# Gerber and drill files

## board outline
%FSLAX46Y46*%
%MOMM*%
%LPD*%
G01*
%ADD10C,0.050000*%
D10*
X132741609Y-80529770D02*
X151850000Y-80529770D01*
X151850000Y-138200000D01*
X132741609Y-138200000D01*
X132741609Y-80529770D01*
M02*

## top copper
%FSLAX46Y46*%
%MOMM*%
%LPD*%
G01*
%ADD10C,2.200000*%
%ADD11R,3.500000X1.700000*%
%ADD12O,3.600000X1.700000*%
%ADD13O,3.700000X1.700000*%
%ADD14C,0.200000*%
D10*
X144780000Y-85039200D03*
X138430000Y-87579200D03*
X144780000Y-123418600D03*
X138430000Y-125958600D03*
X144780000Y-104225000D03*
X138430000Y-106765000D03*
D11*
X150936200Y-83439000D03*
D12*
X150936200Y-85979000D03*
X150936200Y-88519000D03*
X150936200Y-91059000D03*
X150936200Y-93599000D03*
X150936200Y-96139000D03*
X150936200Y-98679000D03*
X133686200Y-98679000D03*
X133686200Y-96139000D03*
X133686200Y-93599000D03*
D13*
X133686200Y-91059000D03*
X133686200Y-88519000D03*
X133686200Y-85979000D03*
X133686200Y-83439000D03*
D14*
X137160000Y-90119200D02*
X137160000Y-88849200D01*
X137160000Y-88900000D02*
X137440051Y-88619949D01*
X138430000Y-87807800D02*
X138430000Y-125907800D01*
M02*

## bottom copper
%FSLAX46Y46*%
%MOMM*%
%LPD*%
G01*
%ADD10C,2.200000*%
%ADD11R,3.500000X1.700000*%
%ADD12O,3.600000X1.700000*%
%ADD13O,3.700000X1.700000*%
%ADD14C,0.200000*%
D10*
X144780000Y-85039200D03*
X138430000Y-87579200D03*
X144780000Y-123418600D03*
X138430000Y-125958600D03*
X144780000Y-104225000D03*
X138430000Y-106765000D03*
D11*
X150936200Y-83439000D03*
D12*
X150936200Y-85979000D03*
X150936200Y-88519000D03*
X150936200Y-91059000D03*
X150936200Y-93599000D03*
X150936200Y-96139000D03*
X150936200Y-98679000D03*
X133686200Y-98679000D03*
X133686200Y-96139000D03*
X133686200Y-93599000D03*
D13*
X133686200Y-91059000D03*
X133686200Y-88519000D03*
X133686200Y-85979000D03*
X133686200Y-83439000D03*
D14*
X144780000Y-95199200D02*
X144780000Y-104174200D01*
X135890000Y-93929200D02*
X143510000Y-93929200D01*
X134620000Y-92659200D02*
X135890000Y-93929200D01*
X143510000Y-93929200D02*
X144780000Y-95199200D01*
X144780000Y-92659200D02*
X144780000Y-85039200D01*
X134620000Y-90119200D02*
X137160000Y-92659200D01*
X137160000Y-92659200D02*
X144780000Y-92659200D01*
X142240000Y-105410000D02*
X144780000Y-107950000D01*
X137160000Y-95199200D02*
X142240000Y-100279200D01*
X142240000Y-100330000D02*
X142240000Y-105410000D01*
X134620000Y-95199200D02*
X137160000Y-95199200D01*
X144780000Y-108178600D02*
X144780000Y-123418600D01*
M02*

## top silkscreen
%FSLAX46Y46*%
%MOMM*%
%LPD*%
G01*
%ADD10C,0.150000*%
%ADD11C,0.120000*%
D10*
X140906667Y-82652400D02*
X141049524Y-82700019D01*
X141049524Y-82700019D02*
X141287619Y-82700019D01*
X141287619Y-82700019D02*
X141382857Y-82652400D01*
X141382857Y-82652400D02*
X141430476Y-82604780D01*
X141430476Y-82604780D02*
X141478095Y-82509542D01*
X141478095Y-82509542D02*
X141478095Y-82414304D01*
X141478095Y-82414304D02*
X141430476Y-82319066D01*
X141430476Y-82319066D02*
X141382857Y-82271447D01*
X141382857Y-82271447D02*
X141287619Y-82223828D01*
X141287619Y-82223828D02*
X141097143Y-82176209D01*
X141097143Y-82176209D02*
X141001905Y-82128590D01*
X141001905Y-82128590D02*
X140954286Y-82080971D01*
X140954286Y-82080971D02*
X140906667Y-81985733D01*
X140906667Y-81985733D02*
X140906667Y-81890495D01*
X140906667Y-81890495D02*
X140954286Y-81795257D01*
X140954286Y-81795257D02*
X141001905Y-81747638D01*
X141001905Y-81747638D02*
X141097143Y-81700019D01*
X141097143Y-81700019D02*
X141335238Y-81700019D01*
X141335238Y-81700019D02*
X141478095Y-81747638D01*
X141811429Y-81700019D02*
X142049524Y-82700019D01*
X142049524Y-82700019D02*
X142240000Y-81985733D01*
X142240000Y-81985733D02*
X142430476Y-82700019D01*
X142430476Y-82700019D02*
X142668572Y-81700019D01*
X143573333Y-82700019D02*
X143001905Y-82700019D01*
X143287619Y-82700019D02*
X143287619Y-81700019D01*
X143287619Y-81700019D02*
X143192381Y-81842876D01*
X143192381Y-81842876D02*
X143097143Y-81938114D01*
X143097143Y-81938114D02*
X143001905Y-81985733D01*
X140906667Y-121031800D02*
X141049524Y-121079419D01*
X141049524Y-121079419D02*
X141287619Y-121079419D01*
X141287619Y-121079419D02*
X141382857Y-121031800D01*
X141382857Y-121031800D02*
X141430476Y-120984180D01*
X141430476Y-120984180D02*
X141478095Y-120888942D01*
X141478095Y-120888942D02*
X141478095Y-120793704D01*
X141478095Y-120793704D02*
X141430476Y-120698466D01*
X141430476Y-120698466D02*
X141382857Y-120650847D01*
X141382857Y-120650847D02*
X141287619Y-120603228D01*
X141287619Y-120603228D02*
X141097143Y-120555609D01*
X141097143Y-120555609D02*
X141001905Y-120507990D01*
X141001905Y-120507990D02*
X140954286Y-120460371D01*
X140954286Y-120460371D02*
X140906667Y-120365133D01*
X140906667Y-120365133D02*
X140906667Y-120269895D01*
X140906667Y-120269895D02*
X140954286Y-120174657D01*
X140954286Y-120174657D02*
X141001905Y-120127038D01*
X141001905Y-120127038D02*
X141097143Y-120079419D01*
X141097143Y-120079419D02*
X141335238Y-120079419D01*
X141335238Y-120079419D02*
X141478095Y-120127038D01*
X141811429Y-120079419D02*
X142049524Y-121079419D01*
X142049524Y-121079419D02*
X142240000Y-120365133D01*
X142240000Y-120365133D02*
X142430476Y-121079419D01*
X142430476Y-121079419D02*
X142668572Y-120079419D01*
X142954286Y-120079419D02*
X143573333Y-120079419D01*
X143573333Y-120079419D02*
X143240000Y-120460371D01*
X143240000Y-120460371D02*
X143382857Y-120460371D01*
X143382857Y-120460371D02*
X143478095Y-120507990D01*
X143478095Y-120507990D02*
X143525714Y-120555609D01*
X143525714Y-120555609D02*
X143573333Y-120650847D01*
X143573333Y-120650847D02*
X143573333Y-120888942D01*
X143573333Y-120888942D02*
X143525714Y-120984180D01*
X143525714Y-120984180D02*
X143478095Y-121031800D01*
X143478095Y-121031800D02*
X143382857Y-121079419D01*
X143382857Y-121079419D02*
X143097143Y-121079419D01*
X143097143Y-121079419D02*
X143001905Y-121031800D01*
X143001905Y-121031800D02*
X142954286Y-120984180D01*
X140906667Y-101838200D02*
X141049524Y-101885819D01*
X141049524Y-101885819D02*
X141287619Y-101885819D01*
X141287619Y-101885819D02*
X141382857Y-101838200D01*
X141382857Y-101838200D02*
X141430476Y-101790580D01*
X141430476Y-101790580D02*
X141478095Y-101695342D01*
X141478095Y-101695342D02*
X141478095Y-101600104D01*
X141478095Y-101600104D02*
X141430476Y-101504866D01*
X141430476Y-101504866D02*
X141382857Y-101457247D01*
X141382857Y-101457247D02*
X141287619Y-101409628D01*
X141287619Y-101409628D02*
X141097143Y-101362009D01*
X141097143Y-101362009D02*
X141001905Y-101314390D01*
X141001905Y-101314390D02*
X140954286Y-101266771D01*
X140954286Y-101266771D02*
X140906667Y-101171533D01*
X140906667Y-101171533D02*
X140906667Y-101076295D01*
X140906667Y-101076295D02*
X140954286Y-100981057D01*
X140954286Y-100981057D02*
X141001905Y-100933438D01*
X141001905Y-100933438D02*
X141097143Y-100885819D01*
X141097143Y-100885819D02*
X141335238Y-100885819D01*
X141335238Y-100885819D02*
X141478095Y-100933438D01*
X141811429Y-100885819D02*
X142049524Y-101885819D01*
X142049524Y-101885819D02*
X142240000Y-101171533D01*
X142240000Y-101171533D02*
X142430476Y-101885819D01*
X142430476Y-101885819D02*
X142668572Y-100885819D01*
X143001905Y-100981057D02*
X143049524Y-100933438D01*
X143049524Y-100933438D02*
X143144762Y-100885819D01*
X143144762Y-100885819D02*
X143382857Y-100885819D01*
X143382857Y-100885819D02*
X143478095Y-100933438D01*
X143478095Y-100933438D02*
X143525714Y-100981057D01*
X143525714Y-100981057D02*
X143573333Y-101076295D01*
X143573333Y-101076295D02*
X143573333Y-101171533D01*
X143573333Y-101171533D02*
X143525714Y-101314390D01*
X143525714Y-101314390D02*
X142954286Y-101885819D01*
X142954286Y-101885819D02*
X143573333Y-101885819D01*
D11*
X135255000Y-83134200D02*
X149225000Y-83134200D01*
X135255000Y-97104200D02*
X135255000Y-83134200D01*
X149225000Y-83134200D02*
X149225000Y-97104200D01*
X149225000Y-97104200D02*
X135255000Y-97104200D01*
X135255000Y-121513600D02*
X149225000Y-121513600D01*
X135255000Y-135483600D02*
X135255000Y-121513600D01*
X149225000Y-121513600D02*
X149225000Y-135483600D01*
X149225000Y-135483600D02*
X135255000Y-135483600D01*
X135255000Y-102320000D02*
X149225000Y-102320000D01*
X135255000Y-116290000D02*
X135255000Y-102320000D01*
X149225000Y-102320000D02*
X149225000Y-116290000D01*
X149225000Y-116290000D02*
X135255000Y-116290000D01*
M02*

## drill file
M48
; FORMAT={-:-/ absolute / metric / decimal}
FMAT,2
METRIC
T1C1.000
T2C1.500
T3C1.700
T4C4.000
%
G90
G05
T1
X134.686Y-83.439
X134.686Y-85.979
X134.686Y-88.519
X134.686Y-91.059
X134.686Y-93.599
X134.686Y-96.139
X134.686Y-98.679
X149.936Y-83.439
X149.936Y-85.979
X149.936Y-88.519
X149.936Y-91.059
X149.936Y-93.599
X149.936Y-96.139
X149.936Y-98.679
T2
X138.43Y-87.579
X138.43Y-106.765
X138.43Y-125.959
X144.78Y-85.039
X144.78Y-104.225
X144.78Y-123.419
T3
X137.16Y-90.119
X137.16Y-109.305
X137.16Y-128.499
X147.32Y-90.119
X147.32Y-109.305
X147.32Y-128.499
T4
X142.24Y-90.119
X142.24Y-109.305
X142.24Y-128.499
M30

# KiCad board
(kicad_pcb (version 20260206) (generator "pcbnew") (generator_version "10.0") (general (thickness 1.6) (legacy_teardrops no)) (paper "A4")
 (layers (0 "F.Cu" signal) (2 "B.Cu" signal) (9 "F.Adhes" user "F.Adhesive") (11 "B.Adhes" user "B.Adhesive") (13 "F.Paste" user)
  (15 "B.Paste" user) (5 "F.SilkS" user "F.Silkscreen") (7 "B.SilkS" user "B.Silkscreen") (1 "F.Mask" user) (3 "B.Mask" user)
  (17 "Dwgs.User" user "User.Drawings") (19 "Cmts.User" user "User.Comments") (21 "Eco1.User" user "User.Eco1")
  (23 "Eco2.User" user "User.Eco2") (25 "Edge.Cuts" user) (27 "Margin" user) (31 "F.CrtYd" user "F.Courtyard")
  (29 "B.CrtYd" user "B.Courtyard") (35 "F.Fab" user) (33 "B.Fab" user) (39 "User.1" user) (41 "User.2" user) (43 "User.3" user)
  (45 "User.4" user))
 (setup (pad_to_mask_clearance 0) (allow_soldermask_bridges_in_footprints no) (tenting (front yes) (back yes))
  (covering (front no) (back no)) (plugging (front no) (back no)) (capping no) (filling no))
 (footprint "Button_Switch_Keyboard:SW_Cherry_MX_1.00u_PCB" (layer "F.Cu") (at 144.78 85.0392)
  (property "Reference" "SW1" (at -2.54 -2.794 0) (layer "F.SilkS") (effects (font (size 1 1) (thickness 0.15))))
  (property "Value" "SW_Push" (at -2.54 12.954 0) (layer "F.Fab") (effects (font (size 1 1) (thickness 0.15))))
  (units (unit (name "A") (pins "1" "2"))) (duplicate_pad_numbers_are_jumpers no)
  (fp_line (start -9.525 -1.905) (end 4.445 -1.905) (stroke (width 0.12) (type solid)) (layer "F.SilkS"))
  (fp_line (start -9.525 12.065) (end -9.525 -1.905) (stroke (width 0.12) (type solid)) (layer "F.SilkS"))
  (fp_line (start 4.445 -1.905) (end 4.445 12.065) (stroke (width 0.12) (type solid)) (layer "F.SilkS"))
  (fp_line (start 4.445 12.065) (end -9.525 12.065) (stroke (width 0.12) (type solid)) (layer "F.SilkS"))
  (pad "" np_thru_hole circle (at -7.62 5.08) (size 1.7 1.7) (drill 1.7) (layers "*.Cu" "*.Mask"))
  (pad "" np_thru_hole circle (at -2.54 5.08) (size 4 4) (drill 4) (layers "*.Cu" "*.Mask"))
  (pad "" np_thru_hole circle (at 2.54 5.08) (size 1.7 1.7) (drill 1.7) (layers "*.Cu" "*.Mask"))
  (pad "1" thru_hole circle (at 0 0) (size 2.2 2.2) (drill 1.5) (layers "*.Cu" "*.Mask") (remove_unused_layers no)
   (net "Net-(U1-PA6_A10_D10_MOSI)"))
  (pad "2" thru_hole circle (at -6.35 2.54) (size 2.2 2.2) (drill 1.5) (layers "*.Cu" "*.Mask") (remove_unused_layers no) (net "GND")))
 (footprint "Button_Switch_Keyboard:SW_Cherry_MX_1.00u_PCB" (layer "F.Cu") (at 144.78 123.4186)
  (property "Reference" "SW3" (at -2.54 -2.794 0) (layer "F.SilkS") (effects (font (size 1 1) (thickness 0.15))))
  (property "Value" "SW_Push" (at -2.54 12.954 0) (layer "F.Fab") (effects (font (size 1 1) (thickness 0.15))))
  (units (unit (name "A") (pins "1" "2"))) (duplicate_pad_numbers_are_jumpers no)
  (fp_line (start -9.525 -1.905) (end 4.445 -1.905) (stroke (width 0.12) (type solid)) (layer "F.SilkS"))
  (fp_line (start -9.525 12.065) (end -9.525 -1.905) (stroke (width 0.12) (type solid)) (layer "F.SilkS"))
  (fp_line (start 4.445 -1.905) (end 4.445 12.065) (stroke (width 0.12) (type solid)) (layer "F.SilkS"))
  (fp_line (start 4.445 12.065) (end -9.525 12.065) (stroke (width 0.12) (type solid)) (layer "F.SilkS"))
  (pad "" np_thru_hole circle (at -7.62 5.08) (size 1.7 1.7) (drill 1.7) (layers "*.Cu" "*.Mask"))
  (pad "" np_thru_hole circle (at -2.54 5.08) (size 4 4) (drill 4) (layers "*.Cu" "*.Mask"))
  (pad "" np_thru_hole circle (at 2.54 5.08) (size 1.7 1.7) (drill 1.7) (layers "*.Cu" "*.Mask"))
  (pad "1" thru_hole circle (at 0 0) (size 2.2 2.2) (drill 1.5) (layers "*.Cu" "*.Mask") (remove_unused_layers no)
   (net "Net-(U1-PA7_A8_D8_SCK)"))
  (pad "2" thru_hole circle (at -6.35 2.54) (size 2.2 2.2) (drill 1.5) (layers "*.Cu" "*.Mask") (remove_unused_layers no) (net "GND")))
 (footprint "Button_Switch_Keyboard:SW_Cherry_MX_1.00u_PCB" (layer "F.Cu") (at 144.78 104.225)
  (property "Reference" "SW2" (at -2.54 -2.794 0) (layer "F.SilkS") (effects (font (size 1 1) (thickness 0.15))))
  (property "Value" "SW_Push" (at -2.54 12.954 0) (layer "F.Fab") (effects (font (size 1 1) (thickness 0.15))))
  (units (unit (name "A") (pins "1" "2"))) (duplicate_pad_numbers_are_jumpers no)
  (fp_line (start -9.525 -1.905) (end 4.445 -1.905) (stroke (width 0.12) (type solid)) (layer "F.SilkS"))
  (fp_line (start -9.525 12.065) (end -9.525 -1.905) (stroke (width 0.12) (type solid)) (layer "F.SilkS"))
  (fp_line (start 4.445 -1.905) (end 4.445 12.065) (stroke (width 0.12) (type solid)) (layer "F.SilkS"))
  (fp_line (start 4.445 12.065) (end -9.525 12.065) (stroke (width 0.12) (type solid)) (layer "F.SilkS"))
  (pad "" np_thru_hole circle (at -7.62 5.08) (size 1.7 1.7) (drill 1.7) (layers "*.Cu" "*.Mask"))
  (pad "" np_thru_hole circle (at -2.54 5.08) (size 4 4) (drill 4) (layers "*.Cu" "*.Mask"))
  (pad "" np_thru_hole circle (at 2.54 5.08) (size 1.7 1.7) (drill 1.7) (layers "*.Cu" "*.Mask"))
  (pad "1" thru_hole circle (at 0 0) (size 2.2 2.2) (drill 1.5) (layers "*.Cu" "*.Mask") (remove_unused_layers no)
   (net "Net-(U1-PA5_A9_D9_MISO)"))
  (pad "2" thru_hole circle (at -6.35 2.54) (size 2.2 2.2) (drill 1.5) (layers "*.Cu" "*.Mask") (remove_unused_layers no) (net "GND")))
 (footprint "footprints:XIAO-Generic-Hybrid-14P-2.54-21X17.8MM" (layer "B.Cu") (at 142.3112 91.059 180)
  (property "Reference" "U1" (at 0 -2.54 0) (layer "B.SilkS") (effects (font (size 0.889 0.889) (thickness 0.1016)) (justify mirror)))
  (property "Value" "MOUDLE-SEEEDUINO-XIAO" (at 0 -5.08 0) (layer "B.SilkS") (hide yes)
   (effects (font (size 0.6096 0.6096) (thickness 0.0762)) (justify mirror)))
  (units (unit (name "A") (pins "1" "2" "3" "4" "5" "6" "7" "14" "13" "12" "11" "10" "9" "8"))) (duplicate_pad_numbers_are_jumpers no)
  (pad "1" thru_hole rect (at -7.625 7.62 180) (size 3.5 1.7) (drill 1 (offset -1 0)) (layers "*.Cu" "*.Mask") (remove_unused_layers no)
   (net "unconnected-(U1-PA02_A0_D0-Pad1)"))
  (pad "2" thru_hole oval (at -7.625 5.08 180) (size 3.6 1.7) (drill 1 (offset -1 0)) (layers "*.Cu" "*.Mask") (remove_unused_layers no)
   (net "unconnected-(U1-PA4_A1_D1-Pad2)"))
  (pad "3" thru_hole oval (at -7.625 2.54 180) (size 3.6 1.7) (drill 1 (offset -1 0)) (layers "*.Cu" "*.Mask") (remove_unused_layers no)
   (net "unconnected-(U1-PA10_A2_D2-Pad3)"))
  (pad "4" thru_hole oval (at -7.625 0 180) (size 3.6 1.7) (drill 1 (offset -1 0)) (layers "*.Cu" "*.Mask") (remove_unused_layers no)
   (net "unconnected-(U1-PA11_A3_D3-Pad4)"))
  (pad "5" thru_hole oval (at -7.625 -2.54 180) (size 3.6 1.7) (drill 1 (offset -1 0)) (layers "*.Cu" "*.Mask") (remove_unused_layers no)
   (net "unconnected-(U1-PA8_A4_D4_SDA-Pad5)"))
  (pad "6" thru_hole oval (at -7.625 -5.08) (size 3.6 1.7) (drill 1 (offset 1 0)) (layers "*.Cu" "*.Mask") (remove_unused_layers no)
   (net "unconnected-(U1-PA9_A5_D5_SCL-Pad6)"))
  (pad "7" thru_hole oval (at -7.625 -7.62 180) (size 3.6 1.7) (drill 1 (offset -1 0)) (layers "*.Cu" "*.Mask") (remove_unused_layers no)
   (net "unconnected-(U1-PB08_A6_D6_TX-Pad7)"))
  (pad "8" thru_hole oval (at 7.625 -7.62 180) (size 3.6 1.7) (drill 1 (offset 1 0)) (layers "*.Cu" "*.Mask") (remove_unused_layers no)
   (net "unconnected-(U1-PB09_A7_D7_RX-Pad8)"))
  (pad "9" thru_hole oval (at 7.625 -5.08 180) (size 3.6 1.7) (drill 1 (offset 1 0)) (layers "*.Cu" "*.Mask") (remove_unused_layers no)
   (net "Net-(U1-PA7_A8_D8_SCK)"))
  (pad "10" thru_hole oval (at 7.625 -2.54 180) (size 3.6 1.7) (drill 1 (offset 1 0)) (layers "*.Cu" "*.Mask") (remove_unused_layers no)
   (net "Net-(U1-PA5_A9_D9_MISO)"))
  (pad "11" thru_hole oval (at 7.625 0 180) (size 3.7 1.7) (drill 1 (offset 1 0)) (layers "*.Cu" "*.Mask") (remove_unused_layers no)
   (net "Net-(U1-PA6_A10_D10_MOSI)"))
  (pad "12" thru_hole oval (at 7.625 2.54 180) (size 3.7 1.7) (drill 1 (offset 1 0)) (layers "*.Cu" "*.Mask") (remove_unused_layers no)
   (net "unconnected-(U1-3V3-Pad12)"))
  (pad "13" thru_hole oval (at 7.625 5.08 180) (size 3.7 1.7) (drill 1 (offset 1 0)) (layers "*.Cu" "*.Mask") (remove_unused_layers no)
   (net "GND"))
  (pad "14" thru_hole oval (at 7.625 7.62 180) (size 3.7 1.7) (drill 1 (offset 1 0)) (layers "*.Cu" "*.Mask") (remove_unused_layers no)
   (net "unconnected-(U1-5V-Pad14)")))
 (gr_rect (start 132.741609 80.52977) (end 151.85 138.2) (stroke (width 0.05) (type default)) (fill no) (layer "Edge.Cuts"))
 (segment (start 137.16 90.1192) (end 137.16 88.8492) (width 0.2) (layer "F.Cu") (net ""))
 (segment (start 137.16 88.9) (end 137.440051 88.619949) (width 0.2) (layer "F.Cu") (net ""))
 (segment (start 144.78 95.1992) (end 144.78 104.1742) (width 0.2) (layer "B.Cu") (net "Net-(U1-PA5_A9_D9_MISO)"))
 (segment (start 135.89 93.9292) (end 143.51 93.9292) (width 0.2) (layer "B.Cu") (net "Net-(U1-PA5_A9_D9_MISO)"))
 (segment (start 134.62 92.6592) (end 135.89 93.9292) (width 0.2) (layer "B.Cu") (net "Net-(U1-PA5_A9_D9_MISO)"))
 (segment (start 143.51 93.9292) (end 144.78 95.1992) (width 0.2) (layer "B.Cu") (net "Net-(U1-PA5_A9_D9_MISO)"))
 (segment (start 138.43 87.8078) (end 138.43 125.9078) (width 0.2) (layer "F.Cu") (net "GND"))
 (segment (start 144.78 92.6592) (end 144.78 85.0392) (width 0.2) (layer "B.Cu") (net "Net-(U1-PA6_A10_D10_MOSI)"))
 (segment (start 134.62 90.1192) (end 137.16 92.6592) (width 0.2) (layer "B.Cu") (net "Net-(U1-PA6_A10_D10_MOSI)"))
 (segment (start 137.16 92.6592) (end 144.78 92.6592) (width 0.2) (layer "B.Cu") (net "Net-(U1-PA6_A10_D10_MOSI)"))
 (segment (start 142.24 105.41) (end 144.78 107.95) (width 0.2) (layer "B.Cu") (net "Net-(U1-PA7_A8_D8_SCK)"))
 (segment (start 137.16 95.1992) (end 142.24 100.2792) (width 0.2) (layer "B.Cu") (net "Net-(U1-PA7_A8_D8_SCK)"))
 (segment (start 142.24 100.33) (end 142.24 105.41) (width 0.2) (layer "B.Cu") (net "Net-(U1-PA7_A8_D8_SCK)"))
 (segment (start 134.62 95.1992) (end 137.16 95.1992) (width 0.2) (layer "B.Cu") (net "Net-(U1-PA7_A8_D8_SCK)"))
 (segment (start 144.78 108.1786) (end 144.78 123.4186) (width 0.2) (layer "B.Cu") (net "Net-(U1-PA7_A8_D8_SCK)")))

